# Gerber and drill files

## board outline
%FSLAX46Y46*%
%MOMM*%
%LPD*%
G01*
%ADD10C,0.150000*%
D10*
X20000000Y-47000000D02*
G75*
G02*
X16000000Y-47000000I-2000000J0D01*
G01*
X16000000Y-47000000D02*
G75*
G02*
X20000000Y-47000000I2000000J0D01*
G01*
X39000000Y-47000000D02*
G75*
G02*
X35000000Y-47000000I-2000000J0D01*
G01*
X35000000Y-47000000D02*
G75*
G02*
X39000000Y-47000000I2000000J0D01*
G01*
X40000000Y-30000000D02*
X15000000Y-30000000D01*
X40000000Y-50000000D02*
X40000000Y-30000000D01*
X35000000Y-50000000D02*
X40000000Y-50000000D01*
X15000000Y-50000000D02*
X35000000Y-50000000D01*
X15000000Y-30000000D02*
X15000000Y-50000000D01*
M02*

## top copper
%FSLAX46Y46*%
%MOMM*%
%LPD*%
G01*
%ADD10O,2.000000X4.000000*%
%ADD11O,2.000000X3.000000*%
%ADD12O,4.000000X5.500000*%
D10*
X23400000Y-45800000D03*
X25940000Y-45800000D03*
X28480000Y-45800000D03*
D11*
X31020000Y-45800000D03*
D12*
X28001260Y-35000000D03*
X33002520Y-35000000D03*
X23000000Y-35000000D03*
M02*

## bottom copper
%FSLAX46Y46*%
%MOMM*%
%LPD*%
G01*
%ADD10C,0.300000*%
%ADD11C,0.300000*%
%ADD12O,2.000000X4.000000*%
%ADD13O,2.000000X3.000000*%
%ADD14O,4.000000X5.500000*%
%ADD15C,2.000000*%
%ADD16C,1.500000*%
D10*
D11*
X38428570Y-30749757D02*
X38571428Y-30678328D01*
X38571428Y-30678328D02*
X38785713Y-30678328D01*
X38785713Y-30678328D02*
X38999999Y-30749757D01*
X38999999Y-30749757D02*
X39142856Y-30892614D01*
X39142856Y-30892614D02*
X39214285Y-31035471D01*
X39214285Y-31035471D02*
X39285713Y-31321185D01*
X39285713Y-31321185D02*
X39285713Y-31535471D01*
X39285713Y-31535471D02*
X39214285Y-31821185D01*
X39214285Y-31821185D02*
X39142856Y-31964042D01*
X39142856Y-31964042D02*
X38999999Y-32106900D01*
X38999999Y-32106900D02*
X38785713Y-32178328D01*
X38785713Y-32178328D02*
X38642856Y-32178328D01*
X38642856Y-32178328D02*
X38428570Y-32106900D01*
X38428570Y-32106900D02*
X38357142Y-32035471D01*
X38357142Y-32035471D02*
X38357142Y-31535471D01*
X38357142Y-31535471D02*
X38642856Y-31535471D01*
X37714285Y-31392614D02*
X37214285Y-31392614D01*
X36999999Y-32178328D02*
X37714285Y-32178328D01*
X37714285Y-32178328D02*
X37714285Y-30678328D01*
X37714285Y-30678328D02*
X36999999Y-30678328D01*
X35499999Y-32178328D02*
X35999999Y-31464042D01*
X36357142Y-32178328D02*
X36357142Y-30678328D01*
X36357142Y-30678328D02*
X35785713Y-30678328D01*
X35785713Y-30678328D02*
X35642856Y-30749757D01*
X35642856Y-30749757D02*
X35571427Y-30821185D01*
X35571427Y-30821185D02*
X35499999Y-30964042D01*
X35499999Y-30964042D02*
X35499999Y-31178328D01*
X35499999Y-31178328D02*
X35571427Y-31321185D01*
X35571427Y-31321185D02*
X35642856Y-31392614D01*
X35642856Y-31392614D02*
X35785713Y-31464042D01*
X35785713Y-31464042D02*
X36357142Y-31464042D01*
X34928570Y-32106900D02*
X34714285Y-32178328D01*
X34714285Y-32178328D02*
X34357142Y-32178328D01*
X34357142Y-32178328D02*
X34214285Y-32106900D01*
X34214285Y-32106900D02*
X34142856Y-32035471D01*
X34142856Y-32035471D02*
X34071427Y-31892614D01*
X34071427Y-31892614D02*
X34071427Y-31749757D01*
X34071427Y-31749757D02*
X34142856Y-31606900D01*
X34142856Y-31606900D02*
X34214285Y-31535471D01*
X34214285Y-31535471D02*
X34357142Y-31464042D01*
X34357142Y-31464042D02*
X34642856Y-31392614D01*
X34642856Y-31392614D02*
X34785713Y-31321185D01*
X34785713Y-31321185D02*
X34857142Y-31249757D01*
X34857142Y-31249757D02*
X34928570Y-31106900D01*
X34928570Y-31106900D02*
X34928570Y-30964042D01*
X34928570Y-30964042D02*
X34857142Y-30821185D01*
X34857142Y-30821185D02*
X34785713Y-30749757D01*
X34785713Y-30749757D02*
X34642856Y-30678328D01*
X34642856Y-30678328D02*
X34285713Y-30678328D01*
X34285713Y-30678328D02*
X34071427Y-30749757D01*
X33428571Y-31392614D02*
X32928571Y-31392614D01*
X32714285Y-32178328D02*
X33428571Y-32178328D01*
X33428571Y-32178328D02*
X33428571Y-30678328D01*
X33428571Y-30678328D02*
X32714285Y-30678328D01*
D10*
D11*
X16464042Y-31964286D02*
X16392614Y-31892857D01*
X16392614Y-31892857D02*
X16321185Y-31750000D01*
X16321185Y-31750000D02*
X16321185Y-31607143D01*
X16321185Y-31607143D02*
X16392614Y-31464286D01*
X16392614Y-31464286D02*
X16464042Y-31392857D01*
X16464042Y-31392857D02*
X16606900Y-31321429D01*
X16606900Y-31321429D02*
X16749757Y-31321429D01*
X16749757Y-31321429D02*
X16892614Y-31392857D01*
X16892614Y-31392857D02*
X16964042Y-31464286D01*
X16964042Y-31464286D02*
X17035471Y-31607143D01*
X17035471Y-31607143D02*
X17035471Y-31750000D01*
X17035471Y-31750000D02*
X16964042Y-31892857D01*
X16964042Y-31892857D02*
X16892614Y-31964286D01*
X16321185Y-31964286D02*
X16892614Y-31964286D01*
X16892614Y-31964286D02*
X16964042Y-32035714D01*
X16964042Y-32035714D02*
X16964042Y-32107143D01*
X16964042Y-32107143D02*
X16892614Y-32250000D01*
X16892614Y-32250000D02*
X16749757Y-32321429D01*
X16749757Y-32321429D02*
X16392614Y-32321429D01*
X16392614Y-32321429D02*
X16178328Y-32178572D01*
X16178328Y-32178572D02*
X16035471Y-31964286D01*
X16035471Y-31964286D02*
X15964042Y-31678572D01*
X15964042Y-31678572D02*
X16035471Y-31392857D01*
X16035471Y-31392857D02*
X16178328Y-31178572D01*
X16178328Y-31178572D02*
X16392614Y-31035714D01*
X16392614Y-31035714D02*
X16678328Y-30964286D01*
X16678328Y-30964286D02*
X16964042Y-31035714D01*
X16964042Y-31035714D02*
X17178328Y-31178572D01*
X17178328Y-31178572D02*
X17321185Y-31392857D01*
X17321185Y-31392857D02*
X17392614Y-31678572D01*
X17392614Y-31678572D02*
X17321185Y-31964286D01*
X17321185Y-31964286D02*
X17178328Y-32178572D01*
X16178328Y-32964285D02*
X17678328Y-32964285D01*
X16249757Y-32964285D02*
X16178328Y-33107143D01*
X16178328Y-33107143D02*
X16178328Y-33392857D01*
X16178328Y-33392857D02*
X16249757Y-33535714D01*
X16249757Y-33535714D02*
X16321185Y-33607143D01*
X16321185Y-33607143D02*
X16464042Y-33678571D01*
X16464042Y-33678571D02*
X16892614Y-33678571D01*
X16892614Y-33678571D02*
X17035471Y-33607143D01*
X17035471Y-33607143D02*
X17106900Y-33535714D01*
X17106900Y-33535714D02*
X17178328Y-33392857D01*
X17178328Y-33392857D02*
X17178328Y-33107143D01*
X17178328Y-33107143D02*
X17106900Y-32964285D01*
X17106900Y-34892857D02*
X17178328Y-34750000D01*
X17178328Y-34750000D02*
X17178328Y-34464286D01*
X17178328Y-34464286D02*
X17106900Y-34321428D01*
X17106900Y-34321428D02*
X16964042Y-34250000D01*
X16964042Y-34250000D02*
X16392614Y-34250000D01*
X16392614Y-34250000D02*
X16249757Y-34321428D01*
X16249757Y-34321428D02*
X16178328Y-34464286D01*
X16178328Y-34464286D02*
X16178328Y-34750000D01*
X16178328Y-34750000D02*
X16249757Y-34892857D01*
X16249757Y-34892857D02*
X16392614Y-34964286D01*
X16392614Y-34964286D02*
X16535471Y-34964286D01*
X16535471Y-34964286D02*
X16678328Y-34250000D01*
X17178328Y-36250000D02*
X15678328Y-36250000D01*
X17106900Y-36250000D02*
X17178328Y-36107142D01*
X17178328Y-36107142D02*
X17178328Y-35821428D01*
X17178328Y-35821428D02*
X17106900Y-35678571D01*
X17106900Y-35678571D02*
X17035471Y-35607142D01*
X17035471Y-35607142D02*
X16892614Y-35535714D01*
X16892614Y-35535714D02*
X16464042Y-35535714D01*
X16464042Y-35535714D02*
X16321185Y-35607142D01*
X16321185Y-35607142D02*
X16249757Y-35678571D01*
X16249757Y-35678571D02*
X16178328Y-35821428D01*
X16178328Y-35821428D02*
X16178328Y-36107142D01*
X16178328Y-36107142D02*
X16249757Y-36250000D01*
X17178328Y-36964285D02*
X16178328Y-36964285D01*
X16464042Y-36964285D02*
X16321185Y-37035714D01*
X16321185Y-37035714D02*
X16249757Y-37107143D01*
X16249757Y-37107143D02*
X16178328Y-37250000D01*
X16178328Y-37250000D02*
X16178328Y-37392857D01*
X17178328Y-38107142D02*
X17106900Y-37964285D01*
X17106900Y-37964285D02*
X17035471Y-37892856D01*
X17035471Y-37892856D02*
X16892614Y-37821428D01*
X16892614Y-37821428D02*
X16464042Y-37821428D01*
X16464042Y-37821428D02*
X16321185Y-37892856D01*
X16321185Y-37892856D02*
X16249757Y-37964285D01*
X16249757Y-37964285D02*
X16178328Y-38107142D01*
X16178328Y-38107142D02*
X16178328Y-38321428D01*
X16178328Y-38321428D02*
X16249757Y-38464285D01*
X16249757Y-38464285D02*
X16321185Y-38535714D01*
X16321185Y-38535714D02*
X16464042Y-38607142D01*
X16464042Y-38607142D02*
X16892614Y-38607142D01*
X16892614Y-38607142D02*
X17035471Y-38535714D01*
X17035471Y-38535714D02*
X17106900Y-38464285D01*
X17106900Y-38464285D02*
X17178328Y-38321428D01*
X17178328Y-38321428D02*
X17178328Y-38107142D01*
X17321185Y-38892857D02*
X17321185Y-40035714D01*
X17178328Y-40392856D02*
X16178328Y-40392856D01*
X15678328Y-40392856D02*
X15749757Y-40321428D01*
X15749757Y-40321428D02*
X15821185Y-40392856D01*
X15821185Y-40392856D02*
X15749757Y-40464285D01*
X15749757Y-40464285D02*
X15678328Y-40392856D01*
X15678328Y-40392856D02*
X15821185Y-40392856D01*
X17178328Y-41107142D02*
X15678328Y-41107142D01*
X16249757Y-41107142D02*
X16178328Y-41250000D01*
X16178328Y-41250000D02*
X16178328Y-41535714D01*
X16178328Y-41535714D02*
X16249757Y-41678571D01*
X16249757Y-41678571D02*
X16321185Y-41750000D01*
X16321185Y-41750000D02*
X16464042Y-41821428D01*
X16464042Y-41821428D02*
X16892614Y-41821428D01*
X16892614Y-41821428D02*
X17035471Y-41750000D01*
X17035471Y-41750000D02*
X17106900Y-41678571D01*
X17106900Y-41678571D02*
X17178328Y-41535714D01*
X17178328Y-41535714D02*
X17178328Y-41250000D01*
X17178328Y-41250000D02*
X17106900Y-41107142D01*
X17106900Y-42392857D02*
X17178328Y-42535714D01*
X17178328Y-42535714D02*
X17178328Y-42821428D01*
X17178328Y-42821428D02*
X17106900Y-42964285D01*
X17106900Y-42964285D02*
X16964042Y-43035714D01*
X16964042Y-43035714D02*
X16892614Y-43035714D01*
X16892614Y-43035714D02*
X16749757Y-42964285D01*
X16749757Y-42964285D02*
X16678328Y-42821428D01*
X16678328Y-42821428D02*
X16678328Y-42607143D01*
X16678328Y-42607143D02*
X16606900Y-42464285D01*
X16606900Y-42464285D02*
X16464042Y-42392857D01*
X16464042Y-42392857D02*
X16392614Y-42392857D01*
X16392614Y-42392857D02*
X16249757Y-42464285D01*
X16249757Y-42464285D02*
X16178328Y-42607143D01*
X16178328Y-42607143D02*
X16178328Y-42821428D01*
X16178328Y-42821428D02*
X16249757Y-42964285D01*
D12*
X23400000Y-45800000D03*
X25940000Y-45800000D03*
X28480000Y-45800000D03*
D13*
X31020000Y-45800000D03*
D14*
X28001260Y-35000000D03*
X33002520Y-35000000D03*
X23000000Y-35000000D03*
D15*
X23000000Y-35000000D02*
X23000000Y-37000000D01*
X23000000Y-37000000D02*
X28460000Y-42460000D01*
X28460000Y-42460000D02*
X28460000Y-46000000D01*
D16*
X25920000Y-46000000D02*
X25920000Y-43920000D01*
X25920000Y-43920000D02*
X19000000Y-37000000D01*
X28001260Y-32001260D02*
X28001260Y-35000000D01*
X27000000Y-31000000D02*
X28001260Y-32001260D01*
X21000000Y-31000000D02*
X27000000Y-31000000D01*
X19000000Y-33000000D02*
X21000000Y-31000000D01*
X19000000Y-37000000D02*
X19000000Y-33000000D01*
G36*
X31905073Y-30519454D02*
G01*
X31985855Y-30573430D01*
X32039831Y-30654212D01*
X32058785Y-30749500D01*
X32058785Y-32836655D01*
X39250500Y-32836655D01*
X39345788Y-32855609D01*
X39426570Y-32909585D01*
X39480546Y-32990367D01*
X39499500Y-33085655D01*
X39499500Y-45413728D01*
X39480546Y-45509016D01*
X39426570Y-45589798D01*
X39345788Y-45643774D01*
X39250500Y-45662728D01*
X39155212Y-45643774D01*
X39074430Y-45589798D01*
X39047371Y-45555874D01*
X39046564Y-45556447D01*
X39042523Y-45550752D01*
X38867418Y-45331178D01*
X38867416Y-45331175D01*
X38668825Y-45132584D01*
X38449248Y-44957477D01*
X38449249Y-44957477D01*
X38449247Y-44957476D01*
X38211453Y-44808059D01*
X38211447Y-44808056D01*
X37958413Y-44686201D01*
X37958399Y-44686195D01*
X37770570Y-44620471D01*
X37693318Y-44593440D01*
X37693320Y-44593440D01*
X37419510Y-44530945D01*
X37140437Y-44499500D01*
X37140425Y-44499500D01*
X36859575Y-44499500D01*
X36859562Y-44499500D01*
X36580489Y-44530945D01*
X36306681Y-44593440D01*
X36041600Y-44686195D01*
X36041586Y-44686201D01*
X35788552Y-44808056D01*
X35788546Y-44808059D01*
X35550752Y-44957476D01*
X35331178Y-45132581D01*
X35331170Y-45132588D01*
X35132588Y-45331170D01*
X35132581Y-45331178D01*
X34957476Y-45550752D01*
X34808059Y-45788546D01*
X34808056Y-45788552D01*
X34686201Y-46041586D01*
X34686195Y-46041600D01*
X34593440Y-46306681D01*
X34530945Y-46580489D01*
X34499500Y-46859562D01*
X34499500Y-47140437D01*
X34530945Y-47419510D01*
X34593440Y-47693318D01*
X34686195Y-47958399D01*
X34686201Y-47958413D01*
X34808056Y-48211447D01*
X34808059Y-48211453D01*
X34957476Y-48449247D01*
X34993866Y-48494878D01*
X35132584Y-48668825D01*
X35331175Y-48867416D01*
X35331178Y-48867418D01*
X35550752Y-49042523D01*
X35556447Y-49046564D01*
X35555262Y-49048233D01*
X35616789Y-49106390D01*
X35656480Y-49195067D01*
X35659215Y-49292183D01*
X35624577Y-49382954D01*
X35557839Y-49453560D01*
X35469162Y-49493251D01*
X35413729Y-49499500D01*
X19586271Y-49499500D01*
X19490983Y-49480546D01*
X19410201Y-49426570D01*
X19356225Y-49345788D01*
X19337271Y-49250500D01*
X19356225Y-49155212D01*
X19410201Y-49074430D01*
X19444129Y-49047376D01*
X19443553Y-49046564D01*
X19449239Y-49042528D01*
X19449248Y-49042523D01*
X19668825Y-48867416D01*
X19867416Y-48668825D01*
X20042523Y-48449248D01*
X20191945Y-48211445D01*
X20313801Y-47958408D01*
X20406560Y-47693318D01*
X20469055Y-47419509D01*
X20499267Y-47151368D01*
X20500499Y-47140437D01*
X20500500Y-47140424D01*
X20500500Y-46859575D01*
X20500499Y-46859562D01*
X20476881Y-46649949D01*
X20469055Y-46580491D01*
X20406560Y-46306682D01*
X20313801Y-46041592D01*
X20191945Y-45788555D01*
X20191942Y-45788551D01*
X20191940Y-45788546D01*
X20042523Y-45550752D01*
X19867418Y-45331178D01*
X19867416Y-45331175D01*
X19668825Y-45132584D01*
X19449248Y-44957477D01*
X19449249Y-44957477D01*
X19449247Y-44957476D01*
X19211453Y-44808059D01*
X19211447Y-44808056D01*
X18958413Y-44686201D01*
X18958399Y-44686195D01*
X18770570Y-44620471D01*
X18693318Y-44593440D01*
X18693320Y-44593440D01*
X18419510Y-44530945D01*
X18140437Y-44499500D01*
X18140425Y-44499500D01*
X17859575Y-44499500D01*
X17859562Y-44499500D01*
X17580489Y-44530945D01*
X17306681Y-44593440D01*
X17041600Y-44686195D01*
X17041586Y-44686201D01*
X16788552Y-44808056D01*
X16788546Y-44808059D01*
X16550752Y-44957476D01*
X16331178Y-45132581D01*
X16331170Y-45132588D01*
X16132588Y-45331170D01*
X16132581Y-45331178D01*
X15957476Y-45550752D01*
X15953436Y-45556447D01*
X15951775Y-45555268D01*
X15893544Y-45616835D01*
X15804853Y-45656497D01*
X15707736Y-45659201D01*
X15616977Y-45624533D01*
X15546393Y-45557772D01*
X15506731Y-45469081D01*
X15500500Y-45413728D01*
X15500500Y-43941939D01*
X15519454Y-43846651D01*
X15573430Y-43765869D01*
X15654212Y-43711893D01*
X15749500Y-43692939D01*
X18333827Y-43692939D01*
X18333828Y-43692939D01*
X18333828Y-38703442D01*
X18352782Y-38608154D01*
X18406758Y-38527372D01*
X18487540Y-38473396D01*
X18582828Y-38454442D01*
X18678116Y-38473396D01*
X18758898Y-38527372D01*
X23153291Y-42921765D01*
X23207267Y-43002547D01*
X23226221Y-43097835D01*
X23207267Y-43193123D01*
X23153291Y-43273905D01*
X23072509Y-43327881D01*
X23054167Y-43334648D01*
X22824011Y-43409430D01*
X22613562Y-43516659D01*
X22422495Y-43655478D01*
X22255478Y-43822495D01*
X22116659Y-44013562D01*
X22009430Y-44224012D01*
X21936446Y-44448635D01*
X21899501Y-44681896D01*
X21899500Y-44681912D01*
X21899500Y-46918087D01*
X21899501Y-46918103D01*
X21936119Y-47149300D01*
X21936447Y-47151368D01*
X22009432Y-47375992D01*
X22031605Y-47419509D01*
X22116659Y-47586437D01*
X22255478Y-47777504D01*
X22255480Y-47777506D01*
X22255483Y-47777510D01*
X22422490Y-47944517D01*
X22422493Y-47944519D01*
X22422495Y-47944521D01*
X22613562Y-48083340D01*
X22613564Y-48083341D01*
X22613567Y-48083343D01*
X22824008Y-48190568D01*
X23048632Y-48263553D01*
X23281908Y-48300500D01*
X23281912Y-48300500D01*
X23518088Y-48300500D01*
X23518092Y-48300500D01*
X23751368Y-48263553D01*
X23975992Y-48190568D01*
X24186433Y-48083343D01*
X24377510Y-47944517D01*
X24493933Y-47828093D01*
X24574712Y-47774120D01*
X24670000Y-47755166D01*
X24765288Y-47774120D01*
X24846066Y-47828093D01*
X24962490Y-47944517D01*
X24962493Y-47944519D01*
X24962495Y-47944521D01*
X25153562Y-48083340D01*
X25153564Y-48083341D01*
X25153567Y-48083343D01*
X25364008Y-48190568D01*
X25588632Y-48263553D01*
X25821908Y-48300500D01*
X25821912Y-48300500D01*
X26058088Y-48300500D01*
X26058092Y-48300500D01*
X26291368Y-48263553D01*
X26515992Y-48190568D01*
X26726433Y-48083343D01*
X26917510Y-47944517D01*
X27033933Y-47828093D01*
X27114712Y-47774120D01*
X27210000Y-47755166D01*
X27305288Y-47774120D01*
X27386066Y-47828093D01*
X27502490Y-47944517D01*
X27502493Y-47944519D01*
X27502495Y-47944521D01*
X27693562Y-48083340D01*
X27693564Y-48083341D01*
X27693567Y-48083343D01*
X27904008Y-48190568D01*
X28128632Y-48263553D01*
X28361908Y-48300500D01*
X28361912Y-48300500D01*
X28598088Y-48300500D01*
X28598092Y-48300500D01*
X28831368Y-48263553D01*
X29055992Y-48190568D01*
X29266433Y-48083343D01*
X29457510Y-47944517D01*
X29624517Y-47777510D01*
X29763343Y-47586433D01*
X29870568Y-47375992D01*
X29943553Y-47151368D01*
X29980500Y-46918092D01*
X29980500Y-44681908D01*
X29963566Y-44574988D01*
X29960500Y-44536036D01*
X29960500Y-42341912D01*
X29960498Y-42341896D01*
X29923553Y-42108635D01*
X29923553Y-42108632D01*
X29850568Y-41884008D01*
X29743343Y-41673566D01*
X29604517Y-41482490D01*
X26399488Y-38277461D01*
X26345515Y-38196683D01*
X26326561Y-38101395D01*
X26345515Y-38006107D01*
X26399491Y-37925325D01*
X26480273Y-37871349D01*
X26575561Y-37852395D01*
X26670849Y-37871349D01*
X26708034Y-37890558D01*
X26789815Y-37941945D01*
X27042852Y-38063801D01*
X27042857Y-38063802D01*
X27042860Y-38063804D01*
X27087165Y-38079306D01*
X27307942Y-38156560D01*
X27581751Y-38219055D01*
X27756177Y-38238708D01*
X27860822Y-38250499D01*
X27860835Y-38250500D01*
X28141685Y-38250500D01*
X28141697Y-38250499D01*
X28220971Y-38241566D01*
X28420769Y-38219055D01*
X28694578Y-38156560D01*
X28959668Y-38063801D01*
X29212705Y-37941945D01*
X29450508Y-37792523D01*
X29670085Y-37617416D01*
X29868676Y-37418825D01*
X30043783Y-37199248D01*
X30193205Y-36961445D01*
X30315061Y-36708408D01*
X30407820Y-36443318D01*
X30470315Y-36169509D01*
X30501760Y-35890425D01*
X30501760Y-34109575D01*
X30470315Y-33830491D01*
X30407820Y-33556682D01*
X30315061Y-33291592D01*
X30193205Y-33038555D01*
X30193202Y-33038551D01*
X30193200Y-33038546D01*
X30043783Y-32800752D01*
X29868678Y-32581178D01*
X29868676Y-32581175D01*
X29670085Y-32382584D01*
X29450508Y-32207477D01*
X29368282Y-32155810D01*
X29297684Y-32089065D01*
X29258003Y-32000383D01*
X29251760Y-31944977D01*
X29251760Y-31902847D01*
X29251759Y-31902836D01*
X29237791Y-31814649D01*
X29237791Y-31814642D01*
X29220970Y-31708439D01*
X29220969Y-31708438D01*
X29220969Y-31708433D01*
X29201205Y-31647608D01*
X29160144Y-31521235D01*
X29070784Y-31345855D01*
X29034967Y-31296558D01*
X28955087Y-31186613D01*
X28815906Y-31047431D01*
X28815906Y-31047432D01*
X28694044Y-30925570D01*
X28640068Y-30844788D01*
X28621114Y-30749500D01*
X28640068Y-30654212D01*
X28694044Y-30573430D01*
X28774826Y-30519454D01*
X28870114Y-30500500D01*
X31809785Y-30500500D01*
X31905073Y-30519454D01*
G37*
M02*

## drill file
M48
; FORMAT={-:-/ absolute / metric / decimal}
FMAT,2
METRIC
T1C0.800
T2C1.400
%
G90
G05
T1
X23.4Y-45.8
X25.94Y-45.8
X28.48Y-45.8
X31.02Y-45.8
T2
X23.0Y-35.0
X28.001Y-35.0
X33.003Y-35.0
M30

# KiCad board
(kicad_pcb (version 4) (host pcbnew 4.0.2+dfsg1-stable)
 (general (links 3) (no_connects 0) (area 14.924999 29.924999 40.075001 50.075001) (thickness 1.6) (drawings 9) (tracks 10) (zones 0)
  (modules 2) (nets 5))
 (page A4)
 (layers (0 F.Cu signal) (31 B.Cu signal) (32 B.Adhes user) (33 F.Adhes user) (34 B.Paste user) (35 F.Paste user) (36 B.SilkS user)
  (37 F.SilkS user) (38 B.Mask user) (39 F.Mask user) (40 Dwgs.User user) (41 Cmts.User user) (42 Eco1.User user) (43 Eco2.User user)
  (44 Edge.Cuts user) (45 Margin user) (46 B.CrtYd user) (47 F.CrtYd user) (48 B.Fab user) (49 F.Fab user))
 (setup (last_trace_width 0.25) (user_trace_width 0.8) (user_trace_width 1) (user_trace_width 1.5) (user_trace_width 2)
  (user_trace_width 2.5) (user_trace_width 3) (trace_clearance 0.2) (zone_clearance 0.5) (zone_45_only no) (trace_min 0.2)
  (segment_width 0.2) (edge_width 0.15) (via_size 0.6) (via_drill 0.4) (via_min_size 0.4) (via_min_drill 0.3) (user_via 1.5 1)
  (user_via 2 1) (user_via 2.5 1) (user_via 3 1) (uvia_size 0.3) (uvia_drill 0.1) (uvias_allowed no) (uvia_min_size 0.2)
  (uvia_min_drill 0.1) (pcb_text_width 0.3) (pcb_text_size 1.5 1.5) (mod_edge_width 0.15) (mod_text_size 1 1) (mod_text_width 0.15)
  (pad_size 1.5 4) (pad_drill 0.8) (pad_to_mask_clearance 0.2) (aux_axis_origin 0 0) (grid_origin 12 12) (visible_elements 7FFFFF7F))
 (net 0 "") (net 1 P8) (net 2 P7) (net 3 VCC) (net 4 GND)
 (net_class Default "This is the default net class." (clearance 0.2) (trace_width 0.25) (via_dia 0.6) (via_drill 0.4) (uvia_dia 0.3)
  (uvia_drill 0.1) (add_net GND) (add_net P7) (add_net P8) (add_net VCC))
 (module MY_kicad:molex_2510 (layer F.Cu) (at 23.4 45.8)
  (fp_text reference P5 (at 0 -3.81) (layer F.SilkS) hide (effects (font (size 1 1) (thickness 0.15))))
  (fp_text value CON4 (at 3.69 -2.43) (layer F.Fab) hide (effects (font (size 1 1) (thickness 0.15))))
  (pad 1 thru_hole oval (at 0 0) (size 2 4) (drill 0.8) (layers *.Cu) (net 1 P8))
  (pad 2 thru_hole oval (at 2.54 0) (size 2 4) (drill 0.8) (layers *.Cu) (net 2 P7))
  (pad 3 thru_hole oval (at 5.08 0) (size 2 4) (drill 0.8) (layers *.Cu) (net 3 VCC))
  (pad 4 thru_hole oval (at 7.62 0) (size 2 3) (drill 0.8) (layers *.Cu) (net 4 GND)))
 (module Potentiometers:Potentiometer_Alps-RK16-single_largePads (layer F.Cu) (at 23 35 90)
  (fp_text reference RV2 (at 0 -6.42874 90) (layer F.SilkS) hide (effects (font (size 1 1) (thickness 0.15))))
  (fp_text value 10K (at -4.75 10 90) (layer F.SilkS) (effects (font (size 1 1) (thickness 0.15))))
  (pad 2 thru_hole oval (at 0 5.00126 90) (size 5.5 4) (drill 1.4) (layers *.Cu) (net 2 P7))
  (pad 3 thru_hole oval (at 0 10.00252 90) (size 5.5 4) (drill 1.4) (layers *.Cu) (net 4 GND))
  (pad 1 thru_hole oval (at 0 0 90) (size 5.5 4) (drill 1.4) (layers *.Cu) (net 3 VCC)))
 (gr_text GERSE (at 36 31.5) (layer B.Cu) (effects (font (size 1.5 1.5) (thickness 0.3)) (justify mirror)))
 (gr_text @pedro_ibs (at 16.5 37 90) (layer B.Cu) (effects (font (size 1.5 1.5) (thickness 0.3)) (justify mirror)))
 (gr_circle (center 18 47) (end 20 47) (layer Edge.Cuts) (width 0.15))
 (gr_circle (center 37 47) (end 39 47) (layer Edge.Cuts) (width 0.15))
 (gr_line (start 40 30) (end 15 30) (angle 90) (layer Edge.Cuts) (width 0.15))
 (gr_line (start 40 50) (end 40 30) (angle 90) (layer Edge.Cuts) (width 0.15))
 (gr_line (start 35 50) (end 40 50) (angle 90) (layer Edge.Cuts) (width 0.15))
 (gr_line (start 15 50) (end 35 50) (angle 90) (layer Edge.Cuts) (width 0.15))
 (gr_line (start 15 30) (end 15 50) (angle 90) (layer Edge.Cuts) (width 0.15))
 (segment (start 23 35) (end 23 37) (width 2) (layer B.Cu) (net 3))
 (segment (start 23 37) (end 28.46 42.46) (width 2) (layer B.Cu) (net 3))
 (segment (start 28.46 42.46) (end 28.46 46) (width 2) (layer B.Cu) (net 3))
 (segment (start 25.92 46) (end 25.92 43.92) (width 1.5) (layer B.Cu) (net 2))
 (segment (start 25.92 43.92) (end 19 37) (width 1.5) (layer B.Cu) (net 2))
 (segment (start 28.00126 32.00126) (end 28.00126 35) (width 1.5) (layer B.Cu) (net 2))
 (segment (start 27 31) (end 28.00126 32.00126) (width 1.5) (layer B.Cu) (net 2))
 (segment (start 21 31) (end 27 31) (width 1.5) (layer B.Cu) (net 2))
 (segment (start 19 33) (end 21 31) (width 1.5) (layer B.Cu) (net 2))
 (segment (start 19 37) (end 19 33) (width 1.5) (layer B.Cu) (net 2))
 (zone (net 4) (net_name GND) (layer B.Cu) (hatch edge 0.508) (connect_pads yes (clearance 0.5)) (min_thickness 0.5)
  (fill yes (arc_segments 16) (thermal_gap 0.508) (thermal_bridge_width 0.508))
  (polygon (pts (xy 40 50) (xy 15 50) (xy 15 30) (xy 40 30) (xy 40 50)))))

